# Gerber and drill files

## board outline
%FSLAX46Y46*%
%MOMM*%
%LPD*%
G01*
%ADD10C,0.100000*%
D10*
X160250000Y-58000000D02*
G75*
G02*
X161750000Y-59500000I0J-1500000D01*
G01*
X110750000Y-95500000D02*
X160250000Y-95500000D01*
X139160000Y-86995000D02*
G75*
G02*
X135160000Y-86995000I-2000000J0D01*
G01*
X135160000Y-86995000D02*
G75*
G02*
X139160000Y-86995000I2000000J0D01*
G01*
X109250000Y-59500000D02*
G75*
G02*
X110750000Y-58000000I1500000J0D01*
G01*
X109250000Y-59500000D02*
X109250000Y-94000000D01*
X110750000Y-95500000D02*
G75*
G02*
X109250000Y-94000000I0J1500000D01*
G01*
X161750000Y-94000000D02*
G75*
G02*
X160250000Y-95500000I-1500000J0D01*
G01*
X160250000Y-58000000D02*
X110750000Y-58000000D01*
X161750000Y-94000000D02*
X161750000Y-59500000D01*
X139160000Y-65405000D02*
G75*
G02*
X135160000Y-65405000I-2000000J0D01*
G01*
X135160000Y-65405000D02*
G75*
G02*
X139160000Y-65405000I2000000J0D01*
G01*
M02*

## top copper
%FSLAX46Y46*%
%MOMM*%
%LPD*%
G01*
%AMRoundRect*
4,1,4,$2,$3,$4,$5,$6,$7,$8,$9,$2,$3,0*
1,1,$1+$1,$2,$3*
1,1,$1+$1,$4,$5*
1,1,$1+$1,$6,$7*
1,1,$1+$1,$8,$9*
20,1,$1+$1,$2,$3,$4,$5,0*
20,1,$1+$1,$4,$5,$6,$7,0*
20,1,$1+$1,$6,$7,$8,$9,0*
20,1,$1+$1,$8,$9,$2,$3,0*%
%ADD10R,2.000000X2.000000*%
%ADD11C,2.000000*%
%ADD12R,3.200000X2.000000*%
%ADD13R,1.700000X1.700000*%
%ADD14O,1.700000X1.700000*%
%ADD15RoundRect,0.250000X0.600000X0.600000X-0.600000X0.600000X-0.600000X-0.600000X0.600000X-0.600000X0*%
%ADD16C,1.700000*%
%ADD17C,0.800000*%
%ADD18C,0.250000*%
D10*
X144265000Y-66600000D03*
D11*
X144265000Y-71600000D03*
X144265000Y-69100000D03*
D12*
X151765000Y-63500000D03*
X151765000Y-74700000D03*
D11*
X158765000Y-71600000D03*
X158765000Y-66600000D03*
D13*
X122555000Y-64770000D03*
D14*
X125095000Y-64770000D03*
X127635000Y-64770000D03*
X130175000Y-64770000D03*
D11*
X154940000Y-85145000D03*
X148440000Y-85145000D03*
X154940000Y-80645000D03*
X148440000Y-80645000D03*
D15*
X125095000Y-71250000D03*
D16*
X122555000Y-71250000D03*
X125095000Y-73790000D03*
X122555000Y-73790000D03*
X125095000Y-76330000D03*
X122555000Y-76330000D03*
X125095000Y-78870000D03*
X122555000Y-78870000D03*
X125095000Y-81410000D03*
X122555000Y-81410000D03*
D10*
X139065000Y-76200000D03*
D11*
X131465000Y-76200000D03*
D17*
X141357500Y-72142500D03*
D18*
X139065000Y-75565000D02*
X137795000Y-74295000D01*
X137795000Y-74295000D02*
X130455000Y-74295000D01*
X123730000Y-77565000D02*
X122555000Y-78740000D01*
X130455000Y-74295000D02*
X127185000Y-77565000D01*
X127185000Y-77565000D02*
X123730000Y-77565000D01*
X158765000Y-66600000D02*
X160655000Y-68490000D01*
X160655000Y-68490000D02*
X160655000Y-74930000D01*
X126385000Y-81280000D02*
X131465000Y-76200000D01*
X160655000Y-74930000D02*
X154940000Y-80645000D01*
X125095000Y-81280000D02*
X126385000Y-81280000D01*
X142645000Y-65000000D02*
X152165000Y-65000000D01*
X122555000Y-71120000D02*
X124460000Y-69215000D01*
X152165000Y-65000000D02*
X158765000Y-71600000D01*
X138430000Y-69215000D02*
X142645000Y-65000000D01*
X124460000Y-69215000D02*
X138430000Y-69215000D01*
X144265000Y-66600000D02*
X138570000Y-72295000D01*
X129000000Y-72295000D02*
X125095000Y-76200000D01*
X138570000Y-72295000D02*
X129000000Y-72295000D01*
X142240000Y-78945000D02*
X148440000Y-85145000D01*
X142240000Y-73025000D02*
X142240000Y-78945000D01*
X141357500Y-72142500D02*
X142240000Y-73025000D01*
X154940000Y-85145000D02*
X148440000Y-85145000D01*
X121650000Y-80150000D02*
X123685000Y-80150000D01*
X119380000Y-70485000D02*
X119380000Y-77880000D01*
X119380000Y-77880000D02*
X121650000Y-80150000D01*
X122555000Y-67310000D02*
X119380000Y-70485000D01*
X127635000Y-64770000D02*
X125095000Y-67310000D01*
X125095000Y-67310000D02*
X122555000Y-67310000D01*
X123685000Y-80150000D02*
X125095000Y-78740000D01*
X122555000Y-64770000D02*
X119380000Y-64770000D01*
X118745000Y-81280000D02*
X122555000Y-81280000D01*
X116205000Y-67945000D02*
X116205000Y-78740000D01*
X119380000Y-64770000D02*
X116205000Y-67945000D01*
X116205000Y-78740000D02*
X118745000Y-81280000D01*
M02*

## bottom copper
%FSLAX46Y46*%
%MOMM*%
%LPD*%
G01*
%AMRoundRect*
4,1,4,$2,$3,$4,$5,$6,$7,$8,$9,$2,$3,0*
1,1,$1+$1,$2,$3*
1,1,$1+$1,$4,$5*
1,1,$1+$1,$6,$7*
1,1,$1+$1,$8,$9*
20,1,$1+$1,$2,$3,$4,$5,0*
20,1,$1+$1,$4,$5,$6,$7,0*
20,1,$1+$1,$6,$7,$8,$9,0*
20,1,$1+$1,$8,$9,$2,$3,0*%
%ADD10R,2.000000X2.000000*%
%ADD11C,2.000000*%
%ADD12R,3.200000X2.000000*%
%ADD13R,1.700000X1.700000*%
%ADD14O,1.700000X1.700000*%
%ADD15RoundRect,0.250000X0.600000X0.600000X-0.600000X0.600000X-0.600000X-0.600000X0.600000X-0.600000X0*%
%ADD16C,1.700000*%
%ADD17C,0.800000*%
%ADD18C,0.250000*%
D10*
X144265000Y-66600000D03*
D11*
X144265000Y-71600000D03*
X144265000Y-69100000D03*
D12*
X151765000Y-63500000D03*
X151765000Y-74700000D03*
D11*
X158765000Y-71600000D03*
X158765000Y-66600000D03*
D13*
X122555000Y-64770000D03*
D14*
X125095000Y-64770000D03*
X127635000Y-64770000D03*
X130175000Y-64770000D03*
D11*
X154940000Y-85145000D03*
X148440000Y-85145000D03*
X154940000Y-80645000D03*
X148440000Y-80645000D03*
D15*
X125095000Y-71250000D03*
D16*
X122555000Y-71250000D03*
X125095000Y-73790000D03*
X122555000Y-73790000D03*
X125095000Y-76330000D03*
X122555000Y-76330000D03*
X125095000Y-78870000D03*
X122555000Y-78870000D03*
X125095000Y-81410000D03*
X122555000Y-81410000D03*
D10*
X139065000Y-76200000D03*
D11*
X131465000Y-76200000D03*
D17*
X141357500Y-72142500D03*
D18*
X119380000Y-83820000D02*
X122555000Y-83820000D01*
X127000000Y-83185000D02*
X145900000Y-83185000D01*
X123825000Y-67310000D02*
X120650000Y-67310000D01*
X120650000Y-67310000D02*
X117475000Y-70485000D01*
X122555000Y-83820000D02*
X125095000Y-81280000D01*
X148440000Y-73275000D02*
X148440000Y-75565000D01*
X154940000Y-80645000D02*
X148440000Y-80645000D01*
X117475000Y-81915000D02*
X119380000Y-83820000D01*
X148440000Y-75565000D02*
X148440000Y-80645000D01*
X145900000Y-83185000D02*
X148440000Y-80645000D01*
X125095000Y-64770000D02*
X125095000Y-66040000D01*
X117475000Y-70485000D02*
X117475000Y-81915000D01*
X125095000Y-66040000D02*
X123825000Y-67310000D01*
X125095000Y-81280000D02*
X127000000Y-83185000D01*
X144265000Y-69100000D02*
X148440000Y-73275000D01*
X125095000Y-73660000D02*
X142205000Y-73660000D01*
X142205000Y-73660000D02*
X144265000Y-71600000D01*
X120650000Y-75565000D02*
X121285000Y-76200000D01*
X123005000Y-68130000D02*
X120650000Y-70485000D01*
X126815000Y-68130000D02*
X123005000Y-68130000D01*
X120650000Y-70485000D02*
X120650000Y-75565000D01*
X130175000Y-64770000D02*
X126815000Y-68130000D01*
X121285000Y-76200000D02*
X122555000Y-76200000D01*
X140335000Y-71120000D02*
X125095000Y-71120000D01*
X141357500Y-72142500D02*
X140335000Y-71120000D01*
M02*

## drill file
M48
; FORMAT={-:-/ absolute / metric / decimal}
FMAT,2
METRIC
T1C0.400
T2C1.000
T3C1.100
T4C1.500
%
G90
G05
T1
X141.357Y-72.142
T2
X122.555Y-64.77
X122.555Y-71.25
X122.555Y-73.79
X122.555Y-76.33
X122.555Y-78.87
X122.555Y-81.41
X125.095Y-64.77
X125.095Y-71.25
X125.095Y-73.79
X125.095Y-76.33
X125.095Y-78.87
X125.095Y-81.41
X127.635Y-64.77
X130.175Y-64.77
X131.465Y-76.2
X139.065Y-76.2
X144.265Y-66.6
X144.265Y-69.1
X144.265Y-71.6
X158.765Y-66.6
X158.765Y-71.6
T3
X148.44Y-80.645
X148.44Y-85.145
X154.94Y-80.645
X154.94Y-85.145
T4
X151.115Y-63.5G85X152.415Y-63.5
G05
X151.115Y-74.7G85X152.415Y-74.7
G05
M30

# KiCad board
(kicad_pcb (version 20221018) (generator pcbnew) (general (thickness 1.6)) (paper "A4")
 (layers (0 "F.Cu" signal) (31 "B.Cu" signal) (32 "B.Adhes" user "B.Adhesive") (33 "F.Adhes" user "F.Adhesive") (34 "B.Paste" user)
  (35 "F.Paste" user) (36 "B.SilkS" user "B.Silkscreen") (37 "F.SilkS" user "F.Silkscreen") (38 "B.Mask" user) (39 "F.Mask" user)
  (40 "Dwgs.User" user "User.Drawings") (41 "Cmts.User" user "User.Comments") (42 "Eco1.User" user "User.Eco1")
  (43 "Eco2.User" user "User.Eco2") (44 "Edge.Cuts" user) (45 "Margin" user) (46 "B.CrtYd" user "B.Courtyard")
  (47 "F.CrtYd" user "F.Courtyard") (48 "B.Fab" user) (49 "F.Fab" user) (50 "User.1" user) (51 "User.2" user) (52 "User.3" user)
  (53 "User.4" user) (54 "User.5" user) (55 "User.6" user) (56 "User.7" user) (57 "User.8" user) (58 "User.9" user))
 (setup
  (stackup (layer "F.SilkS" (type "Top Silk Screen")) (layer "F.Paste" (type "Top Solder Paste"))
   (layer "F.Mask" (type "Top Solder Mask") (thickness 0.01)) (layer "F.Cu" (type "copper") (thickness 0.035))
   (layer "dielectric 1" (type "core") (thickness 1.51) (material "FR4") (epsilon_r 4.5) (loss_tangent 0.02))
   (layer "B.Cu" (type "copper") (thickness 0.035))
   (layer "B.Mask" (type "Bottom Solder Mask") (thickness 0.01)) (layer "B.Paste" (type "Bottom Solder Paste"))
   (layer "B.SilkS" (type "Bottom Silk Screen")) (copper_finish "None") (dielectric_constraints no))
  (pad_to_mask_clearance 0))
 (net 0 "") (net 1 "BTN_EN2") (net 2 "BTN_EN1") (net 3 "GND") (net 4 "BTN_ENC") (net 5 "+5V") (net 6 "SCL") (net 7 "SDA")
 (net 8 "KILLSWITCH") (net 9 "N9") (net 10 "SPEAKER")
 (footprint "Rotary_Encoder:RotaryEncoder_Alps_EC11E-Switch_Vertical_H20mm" (layer "F.Cu") (at 144.265 66.6)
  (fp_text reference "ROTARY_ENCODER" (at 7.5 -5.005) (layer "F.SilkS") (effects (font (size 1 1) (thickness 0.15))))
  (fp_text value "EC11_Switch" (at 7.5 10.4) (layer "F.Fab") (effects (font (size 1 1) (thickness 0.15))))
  (pad "A" thru_hole rect (at 0 0) (size 2 2) (drill 1) (layers "*.Cu" "*.Mask") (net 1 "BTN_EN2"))
  (pad "B" thru_hole circle (at 0 5) (size 2 2) (drill 1) (layers "*.Cu" "*.Mask") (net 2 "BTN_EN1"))
  (pad "C" thru_hole circle (at 0 2.5) (size 2 2) (drill 1) (layers "*.Cu" "*.Mask") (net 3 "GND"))
  (pad "MP" thru_hole rect (at 7.5 -3.1) (size 3.2 2) (drill oval 2.8 1.5) (layers "*.Cu" "*.Mask"))
  (pad "MP" thru_hole rect (at 7.5 8.1) (size 3.2 2) (drill oval 2.8 1.5) (layers "*.Cu" "*.Mask"))
  (pad "S1" thru_hole circle (at 14.5 5) (size 2 2) (drill 1) (layers "*.Cu" "*.Mask") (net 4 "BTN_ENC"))
  (pad "S2" thru_hole circle (at 14.5 0) (size 2 2) (drill 1) (layers "*.Cu" "*.Mask") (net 3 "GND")))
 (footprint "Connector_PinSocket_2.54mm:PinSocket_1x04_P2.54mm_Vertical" (layer "F.Cu") (at 122.555 64.77 90)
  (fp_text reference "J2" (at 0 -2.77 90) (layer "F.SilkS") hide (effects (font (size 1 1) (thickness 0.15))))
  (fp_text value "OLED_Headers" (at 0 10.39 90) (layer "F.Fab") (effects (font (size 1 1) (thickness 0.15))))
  (pad "1" thru_hole rect (at 0 0 90) (size 1.7 1.7) (drill 1) (layers "*.Cu" "*.Mask") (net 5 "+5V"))
  (pad "2" thru_hole oval (at 0 2.54 90) (size 1.7 1.7) (drill 1) (layers "*.Cu" "*.Mask") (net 3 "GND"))
  (pad "3" thru_hole oval (at 0 5.08 90) (size 1.7 1.7) (drill 1) (layers "*.Cu" "*.Mask") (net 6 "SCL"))
  (pad "4" thru_hole oval (at 0 7.62 90) (size 1.7 1.7) (drill 1) (layers "*.Cu" "*.Mask") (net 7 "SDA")))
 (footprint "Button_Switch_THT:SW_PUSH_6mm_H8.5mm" (layer "F.Cu") (at 154.94 85.145 180)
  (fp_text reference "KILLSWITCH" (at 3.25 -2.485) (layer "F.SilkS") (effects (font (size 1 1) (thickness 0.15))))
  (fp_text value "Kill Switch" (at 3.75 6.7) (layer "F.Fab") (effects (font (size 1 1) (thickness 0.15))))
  (pad "1" thru_hole circle (at 0 0 270) (size 2 2) (drill 1.1) (layers "*.Cu" "*.Mask") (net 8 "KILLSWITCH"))
  (pad "1" thru_hole circle (at 6.5 0 270) (size 2 2) (drill 1.1) (layers "*.Cu" "*.Mask") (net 8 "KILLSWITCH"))
  (pad "2" thru_hole circle (at 0 4.5 270) (size 2 2) (drill 1.1) (layers "*.Cu" "*.Mask") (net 3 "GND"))
  (pad "2" thru_hole circle (at 6.5 4.5 270) (size 2 2) (drill 1.1) (layers "*.Cu" "*.Mask") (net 3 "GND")))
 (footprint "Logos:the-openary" (layer "F.Cu") (at 150.5 91.75)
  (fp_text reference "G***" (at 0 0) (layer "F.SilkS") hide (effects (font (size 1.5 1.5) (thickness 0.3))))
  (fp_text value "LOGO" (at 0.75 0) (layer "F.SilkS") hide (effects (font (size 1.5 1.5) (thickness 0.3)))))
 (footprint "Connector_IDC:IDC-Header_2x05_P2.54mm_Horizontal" (layer "B.Cu") (at 125.095 71.25 180)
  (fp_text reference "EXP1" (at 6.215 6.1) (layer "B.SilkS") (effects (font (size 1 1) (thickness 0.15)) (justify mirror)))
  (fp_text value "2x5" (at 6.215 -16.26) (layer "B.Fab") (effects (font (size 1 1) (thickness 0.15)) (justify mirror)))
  (pad "1" thru_hole roundrect (at 0 0 180) (size 1.7 1.7) (drill 1) (layers "*.Cu" "*.Mask") (roundrect_rratio 0.1470588235)
   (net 8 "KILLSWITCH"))
  (pad "2" thru_hole circle (at 2.54 0 180) (size 1.7 1.7) (drill 1) (layers "*.Cu" "*.Mask") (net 4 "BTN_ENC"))
  (pad "3" thru_hole circle (at 0 -2.54 180) (size 1.7 1.7) (drill 1) (layers "*.Cu" "*.Mask") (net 2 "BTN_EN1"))
  (pad "4" thru_hole circle (at 2.54 -2.54 180) (size 1.7 1.7) (drill 1) (layers "*.Cu" "*.Mask") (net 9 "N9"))
  (pad "5" thru_hole circle (at 0 -5.08 180) (size 1.7 1.7) (drill 1) (layers "*.Cu" "*.Mask") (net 1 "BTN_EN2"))
  (pad "6" thru_hole circle (at 2.54 -5.08 180) (size 1.7 1.7) (drill 1) (layers "*.Cu" "*.Mask") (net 7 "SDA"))
  (pad "7" thru_hole circle (at 0 -7.62 180) (size 1.7 1.7) (drill 1) (layers "*.Cu" "*.Mask") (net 6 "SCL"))
  (pad "8" thru_hole circle (at 2.54 -7.62 180) (size 1.7 1.7) (drill 1) (layers "*.Cu" "*.Mask") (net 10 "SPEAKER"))
  (pad "9" thru_hole circle (at 0 -10.16 180) (size 1.7 1.7) (drill 1) (layers "*.Cu" "*.Mask") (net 3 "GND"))
  (pad "10" thru_hole circle (at 2.54 -10.16 180) (size 1.7 1.7) (drill 1) (layers "*.Cu" "*.Mask") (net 5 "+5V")))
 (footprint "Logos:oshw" (layer "B.Cu") (at 129.25 89.75 180)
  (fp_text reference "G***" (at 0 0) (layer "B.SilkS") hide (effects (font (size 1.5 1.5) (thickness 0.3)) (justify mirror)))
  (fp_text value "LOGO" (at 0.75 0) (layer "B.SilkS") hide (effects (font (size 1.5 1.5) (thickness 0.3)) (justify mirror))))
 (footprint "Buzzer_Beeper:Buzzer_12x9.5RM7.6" (layer "B.Cu") (at 139.065 76.2 180)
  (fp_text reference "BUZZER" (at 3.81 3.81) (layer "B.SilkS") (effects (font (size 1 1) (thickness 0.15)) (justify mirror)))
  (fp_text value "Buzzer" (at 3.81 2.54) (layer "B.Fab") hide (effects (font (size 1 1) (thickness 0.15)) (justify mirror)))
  (pad "1" thru_hole rect (at 0 0 180) (size 2 2) (drill 1) (layers "*.Cu" "*.Mask") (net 10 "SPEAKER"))
  (pad "2" thru_hole circle (at 7.6 0 180) (size 2 2) (drill 1) (layers "*.Cu" "*.Mask") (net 3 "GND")))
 (gr_arc (start 160.25 58) (mid 161.31066 58.43934) (end 161.75 59.5) (stroke (width 0.1) (type default)) (layer "Edge.Cuts"))
 (gr_line (start 110.75 95.5) (end 160.25 95.5) (stroke (width 0.1) (type default)) (layer "Edge.Cuts"))
 (gr_circle (center 137.16 86.995) (end 139.16 86.995) (stroke (width 0.1) (type default)) (fill none) (layer "Edge.Cuts"))
 (gr_arc (start 109.25 59.5) (mid 109.68934 58.43934) (end 110.75 58) (stroke (width 0.1) (type default)) (layer "Edge.Cuts"))
 (gr_line (start 109.25 59.5) (end 109.25 94) (stroke (width 0.1) (type default)) (layer "Edge.Cuts"))
 (gr_arc (start 110.75 95.5) (mid 109.68934 95.06066) (end 109.25 94) (stroke (width 0.1) (type default)) (layer "Edge.Cuts"))
 (gr_arc (start 161.75 94) (mid 161.31066 95.06066) (end 160.25 95.5) (stroke (width 0.1) (type default)) (layer "Edge.Cuts"))
 (gr_line (start 160.25 58) (end 110.75 58) (stroke (width 0.1) (type default)) (layer "Edge.Cuts"))
 (gr_line (start 161.75 94) (end 161.75 59.5) (stroke (width 0.1) (type default)) (layer "Edge.Cuts"))
 (gr_circle (center 137.16 65.405) (end 139.16 65.405) (stroke (width 0.1) (type default)) (fill none) (layer "Edge.Cuts"))
 (segment (start 139.065 75.565) (end 137.795 74.295) (width 0.25) (layer "F.Cu") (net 10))
 (segment (start 137.795 74.295) (end 130.455 74.295) (width 0.25) (layer "F.Cu") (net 10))
 (segment (start 123.73 77.565) (end 122.555 78.74) (width 0.25) (layer "F.Cu") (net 10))
 (segment (start 130.455 74.295) (end 127.185 77.565) (width 0.25) (layer "F.Cu") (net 10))
 (segment (start 127.185 77.565) (end 123.73 77.565) (width 0.25) (layer "F.Cu") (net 10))
 (segment (start 158.765 66.6) (end 160.655 68.49) (width 0.25) (layer "F.Cu") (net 3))
 (segment (start 160.655 68.49) (end 160.655 74.93) (width 0.25) (layer "F.Cu") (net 3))
 (segment (start 126.385 81.28) (end 131.465 76.2) (width 0.25) (layer "F.Cu") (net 3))
 (segment (start 160.655 74.93) (end 154.94 80.645) (width 0.25) (layer "F.Cu") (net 3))
 (segment (start 125.095 81.28) (end 126.385 81.28) (width 0.25) (layer "F.Cu") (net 3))
 (segment (start 119.38 83.82) (end 122.555 83.82) (width 0.25) (layer "B.Cu") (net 3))
 (segment (start 127 83.185) (end 145.9 83.185) (width 0.25) (layer "B.Cu") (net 3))
 (segment (start 123.825 67.31) (end 120.65 67.31) (width 0.25) (layer "B.Cu") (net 3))
 (segment (start 120.65 67.31) (end 117.475 70.485) (width 0.25) (layer "B.Cu") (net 3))
 (segment (start 122.555 83.82) (end 125.095 81.28) (width 0.25) (layer "B.Cu") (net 3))
 (segment (start 148.44 73.275) (end 148.44 75.565) (width 0.25) (layer "B.Cu") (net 3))
 (segment (start 154.94 80.645) (end 148.44 80.645) (width 0.25) (layer "B.Cu") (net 3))
 (segment (start 117.475 81.915) (end 119.38 83.82) (width 0.25) (layer "B.Cu") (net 3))
 (segment (start 148.44 75.565) (end 148.44 80.645) (width 0.25) (layer "B.Cu") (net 3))
 (segment (start 145.9 83.185) (end 148.44 80.645) (width 0.25) (layer "B.Cu") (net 3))
 (segment (start 125.095 64.77) (end 125.095 66.04) (width 0.25) (layer "B.Cu") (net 3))
 (segment (start 117.475 70.485) (end 117.475 81.915) (width 0.25) (layer "B.Cu") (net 3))
 (segment (start 125.095 66.04) (end 123.825 67.31) (width 0.25) (layer "B.Cu") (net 3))
 (segment (start 125.095 81.28) (end 127 83.185) (width 0.25) (layer "B.Cu") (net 3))
 (segment (start 144.265 69.1) (end 148.44 73.275) (width 0.25) (layer "B.Cu") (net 3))
 (segment (start 142.645 65) (end 152.165 65) (width 0.25) (layer "F.Cu") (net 4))
 (segment (start 122.555 71.12) (end 124.46 69.215) (width 0.25) (layer "F.Cu") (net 4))
 (segment (start 152.165 65) (end 158.765 71.6) (width 0.25) (layer "F.Cu") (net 4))
 (segment (start 138.43 69.215) (end 142.645 65) (width 0.25) (layer "F.Cu") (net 4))
 (segment (start 124.46 69.215) (end 138.43 69.215) (width 0.25) (layer "F.Cu") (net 4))
 (segment (start 125.095 73.66) (end 142.205 73.66) (width 0.25) (layer "B.Cu") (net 2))
 (segment (start 142.205 73.66) (end 144.265 71.6) (width 0.25) (layer "B.Cu") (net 2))
 (segment (start 144.265 66.6) (end 138.57 72.295) (width 0.25) (layer "F.Cu") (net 1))
 (segment (start 129 72.295) (end 125.095 76.2) (width 0.25) (layer "F.Cu") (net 1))
 (segment (start 138.57 72.295) (end 129 72.295) (width 0.25) (layer "F.Cu") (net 1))
 (segment (start 120.65 75.565) (end 121.285 76.2) (width 0.25) (layer "B.Cu") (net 7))
 (segment (start 123.005 68.13) (end 120.65 70.485) (width 0.25) (layer "B.Cu") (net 7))
 (segment (start 126.815 68.13) (end 123.005 68.13) (width 0.25) (layer "B.Cu") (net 7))
 (segment (start 120.65 70.485) (end 120.65 75.565) (width 0.25) (layer "B.Cu") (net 7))
 (segment (start 130.175 64.77) (end 126.815 68.13) (width 0.25) (layer "B.Cu") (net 7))
 (segment (start 121.285 76.2) (end 122.555 76.2) (width 0.25) (layer "B.Cu") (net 7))
 (segment (start 142.24 78.945) (end 148.44 85.145) (width 0.25) (layer "F.Cu") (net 8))
 (segment (start 142.24 73.025) (end 142.24 78.945) (width 0.25) (layer "F.Cu") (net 8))
 (segment (start 141.3575 72.1425) (end 142.24 73.025) (width 0.25) (layer "F.Cu") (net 8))
 (segment (start 154.94 85.145) (end 148.44 85.145) (width 0.25) (layer "F.Cu") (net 8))
 (via (at 141.3575 72.1425) (size 0.8) (drill 0.4) (layers "F.Cu" "B.Cu") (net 8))
 (segment (start 140.335 71.12) (end 125.095 71.12) (width 0.25) (layer "B.Cu") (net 8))
 (segment (start 141.3575 72.1425) (end 140.335 71.12) (width 0.25) (layer "B.Cu") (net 8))
 (segment (start 121.65 80.15) (end 123.685 80.15) (width 0.25) (layer "F.Cu") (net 6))
 (segment (start 119.38 70.485) (end 119.38 77.88) (width 0.25) (layer "F.Cu") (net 6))
 (segment (start 119.38 77.88) (end 121.65 80.15) (width 0.25) (layer "F.Cu") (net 6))
 (segment (start 122.555 67.31) (end 119.38 70.485) (width 0.25) (layer "F.Cu") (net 6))
 (segment (start 127.635 64.77) (end 125.095 67.31) (width 0.25) (layer "F.Cu") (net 6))
 (segment (start 125.095 67.31) (end 122.555 67.31) (width 0.25) (layer "F.Cu") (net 6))
 (segment (start 123.685 80.15) (end 125.095 78.74) (width 0.25) (layer "F.Cu") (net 6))
 (segment (start 122.555 64.77) (end 119.38 64.77) (width 0.25) (layer "F.Cu") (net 5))
 (segment (start 118.745 81.28) (end 122.555 81.28) (width 0.25) (layer "F.Cu") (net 5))
 (segment (start 116.205 67.945) (end 116.205 78.74) (width 0.25) (layer "F.Cu") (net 5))
 (segment (start 119.38 64.77) (end 116.205 67.945) (width 0.25) (layer "F.Cu") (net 5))
 (segment (start 116.205 78.74) (end 118.745 81.28) (width 0.25) (layer "F.Cu") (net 5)))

